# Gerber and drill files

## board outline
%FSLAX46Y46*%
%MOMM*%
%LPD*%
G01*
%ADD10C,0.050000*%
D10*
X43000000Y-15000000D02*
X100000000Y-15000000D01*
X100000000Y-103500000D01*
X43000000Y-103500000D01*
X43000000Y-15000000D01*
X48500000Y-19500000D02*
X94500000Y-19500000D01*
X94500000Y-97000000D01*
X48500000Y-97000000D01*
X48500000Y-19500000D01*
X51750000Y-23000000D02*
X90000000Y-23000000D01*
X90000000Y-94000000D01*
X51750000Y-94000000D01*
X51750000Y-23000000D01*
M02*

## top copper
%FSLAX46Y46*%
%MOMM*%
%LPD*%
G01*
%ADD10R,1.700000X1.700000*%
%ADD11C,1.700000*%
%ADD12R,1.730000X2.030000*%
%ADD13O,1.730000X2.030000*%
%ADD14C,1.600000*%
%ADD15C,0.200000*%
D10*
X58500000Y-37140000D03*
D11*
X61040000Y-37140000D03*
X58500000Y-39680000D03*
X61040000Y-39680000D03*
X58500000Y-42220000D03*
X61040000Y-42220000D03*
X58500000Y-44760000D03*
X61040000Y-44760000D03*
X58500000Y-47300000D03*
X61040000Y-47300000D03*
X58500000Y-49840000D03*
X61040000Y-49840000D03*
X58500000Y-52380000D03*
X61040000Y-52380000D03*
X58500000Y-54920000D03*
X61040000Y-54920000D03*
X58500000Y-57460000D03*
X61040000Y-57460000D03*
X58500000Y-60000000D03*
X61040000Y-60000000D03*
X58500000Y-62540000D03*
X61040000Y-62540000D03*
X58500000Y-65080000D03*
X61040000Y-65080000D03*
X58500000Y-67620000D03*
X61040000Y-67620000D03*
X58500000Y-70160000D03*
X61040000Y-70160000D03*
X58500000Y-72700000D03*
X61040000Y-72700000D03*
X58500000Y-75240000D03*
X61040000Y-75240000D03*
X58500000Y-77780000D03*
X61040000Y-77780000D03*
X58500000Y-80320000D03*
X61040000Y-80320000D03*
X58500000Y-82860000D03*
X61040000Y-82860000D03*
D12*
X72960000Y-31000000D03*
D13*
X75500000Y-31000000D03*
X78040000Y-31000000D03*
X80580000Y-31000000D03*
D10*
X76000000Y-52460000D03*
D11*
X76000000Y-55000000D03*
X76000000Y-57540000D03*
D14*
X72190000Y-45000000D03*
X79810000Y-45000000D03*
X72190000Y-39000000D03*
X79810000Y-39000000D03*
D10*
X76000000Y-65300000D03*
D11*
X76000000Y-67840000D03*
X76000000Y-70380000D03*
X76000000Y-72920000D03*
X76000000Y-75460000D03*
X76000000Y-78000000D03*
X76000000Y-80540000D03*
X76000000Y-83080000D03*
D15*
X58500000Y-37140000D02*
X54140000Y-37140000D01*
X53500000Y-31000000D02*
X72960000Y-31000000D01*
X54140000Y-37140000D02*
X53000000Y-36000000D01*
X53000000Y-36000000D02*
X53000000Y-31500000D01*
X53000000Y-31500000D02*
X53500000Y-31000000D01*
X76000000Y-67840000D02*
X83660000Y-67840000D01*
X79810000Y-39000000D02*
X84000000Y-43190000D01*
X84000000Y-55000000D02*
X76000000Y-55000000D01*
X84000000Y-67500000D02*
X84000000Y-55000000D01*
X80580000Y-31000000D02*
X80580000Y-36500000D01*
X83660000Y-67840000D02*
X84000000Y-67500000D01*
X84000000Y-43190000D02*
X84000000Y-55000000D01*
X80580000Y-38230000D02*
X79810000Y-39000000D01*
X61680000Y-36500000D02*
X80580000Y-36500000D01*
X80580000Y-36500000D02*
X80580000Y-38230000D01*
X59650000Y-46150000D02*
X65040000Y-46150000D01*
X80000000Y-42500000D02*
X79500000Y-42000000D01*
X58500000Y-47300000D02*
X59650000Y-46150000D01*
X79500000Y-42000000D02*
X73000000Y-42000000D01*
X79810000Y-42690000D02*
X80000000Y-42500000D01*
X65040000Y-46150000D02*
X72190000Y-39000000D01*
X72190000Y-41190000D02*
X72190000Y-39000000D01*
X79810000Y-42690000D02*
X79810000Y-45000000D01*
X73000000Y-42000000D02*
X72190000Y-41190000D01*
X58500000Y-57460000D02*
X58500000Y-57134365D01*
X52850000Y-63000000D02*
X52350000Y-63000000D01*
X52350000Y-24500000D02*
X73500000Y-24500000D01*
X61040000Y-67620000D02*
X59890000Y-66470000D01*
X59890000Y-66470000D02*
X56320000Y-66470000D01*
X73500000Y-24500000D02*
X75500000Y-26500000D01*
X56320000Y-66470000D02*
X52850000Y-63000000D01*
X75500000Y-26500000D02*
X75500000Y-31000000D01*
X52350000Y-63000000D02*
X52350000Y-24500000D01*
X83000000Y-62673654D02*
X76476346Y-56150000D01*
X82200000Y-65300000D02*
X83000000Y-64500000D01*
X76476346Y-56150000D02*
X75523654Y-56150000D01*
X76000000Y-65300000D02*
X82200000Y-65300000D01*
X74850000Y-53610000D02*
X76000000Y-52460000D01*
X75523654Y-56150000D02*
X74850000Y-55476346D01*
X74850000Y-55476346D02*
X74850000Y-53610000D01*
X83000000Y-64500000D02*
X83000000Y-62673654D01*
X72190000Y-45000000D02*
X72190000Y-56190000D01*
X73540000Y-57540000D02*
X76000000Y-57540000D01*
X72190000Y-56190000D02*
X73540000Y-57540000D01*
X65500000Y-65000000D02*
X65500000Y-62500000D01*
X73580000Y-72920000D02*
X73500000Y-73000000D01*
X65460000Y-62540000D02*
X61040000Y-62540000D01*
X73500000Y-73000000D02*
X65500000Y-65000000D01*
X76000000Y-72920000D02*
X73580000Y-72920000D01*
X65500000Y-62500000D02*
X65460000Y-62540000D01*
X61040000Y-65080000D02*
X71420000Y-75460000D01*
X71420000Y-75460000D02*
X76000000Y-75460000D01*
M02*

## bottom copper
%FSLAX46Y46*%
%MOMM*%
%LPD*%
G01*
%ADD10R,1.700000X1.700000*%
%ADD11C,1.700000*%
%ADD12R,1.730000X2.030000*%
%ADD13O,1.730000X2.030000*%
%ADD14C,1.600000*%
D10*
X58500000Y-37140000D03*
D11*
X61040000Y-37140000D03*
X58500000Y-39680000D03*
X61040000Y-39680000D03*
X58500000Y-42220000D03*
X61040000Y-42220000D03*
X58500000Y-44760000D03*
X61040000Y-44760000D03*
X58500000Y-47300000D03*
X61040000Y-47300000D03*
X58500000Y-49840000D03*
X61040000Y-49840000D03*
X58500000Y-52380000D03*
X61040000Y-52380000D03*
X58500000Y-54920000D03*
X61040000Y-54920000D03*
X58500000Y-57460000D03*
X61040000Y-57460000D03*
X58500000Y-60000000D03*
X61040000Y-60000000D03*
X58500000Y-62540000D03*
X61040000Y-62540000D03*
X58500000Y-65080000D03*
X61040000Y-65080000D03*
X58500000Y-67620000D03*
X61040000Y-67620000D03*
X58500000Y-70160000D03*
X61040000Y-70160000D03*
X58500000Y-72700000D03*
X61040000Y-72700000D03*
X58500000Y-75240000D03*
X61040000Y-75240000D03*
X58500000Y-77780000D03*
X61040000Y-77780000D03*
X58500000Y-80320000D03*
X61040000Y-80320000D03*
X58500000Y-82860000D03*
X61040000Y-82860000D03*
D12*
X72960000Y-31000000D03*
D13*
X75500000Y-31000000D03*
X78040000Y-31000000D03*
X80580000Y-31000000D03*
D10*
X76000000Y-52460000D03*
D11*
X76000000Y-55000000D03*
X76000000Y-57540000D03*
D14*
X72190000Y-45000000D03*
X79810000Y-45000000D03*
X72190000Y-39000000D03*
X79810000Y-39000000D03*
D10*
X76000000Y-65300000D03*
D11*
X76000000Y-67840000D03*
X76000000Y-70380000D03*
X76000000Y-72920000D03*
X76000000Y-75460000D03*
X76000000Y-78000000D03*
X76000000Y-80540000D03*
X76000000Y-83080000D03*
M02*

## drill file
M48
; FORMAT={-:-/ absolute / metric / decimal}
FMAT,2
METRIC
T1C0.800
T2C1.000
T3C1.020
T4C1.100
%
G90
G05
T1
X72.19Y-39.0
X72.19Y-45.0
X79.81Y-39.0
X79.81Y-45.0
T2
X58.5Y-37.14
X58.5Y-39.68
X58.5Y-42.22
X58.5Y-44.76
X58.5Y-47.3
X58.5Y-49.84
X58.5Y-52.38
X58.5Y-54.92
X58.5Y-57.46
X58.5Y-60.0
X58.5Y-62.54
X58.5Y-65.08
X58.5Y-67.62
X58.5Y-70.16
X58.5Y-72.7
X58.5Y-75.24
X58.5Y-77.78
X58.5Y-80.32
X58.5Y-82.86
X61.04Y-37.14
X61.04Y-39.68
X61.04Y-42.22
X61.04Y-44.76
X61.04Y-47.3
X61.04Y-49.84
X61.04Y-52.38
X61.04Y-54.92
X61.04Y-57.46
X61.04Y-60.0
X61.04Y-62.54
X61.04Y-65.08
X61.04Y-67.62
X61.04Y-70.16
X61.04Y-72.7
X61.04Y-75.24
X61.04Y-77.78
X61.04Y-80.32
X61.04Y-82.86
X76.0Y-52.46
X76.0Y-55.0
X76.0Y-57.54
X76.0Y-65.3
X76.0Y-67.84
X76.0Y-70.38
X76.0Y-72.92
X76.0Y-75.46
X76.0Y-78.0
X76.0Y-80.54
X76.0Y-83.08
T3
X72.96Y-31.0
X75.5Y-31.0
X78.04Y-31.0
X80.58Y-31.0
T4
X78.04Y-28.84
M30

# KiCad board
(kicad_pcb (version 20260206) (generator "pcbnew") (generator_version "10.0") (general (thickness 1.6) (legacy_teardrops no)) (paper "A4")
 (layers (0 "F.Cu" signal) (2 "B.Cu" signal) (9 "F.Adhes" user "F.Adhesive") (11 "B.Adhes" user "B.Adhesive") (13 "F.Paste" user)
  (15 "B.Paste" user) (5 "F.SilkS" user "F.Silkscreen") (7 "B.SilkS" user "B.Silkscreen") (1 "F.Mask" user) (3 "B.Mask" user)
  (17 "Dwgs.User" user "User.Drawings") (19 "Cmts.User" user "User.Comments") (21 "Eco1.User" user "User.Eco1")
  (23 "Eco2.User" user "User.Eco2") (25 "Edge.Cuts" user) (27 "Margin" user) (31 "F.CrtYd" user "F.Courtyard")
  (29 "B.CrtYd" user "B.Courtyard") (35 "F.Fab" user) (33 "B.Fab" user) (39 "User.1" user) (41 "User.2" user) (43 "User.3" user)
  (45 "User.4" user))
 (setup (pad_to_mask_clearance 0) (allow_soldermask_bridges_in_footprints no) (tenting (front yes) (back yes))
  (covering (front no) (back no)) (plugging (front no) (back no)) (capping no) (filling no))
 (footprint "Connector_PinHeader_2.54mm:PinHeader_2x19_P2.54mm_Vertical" (layer "F.Cu") (at 58.5 37.14)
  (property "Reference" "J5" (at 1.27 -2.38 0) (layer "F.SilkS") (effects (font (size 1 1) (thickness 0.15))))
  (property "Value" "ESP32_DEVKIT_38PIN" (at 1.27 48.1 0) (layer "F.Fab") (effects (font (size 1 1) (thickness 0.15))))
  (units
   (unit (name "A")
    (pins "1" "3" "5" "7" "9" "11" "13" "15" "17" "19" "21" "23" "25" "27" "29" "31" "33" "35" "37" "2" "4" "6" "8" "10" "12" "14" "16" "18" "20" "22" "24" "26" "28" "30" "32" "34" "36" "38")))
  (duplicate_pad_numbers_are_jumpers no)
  (pad "1" thru_hole rect (at 0 0) (size 1.7 1.7) (drill 1) (layers "*.Cu" "*.Mask") (remove_unused_layers no) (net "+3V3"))
  (pad "2" thru_hole circle (at 2.54 0) (size 1.7 1.7) (drill 1) (layers "*.Cu" "*.Mask") (remove_unused_layers no) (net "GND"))
  (pad "3" thru_hole circle (at 0 2.54) (size 1.7 1.7) (drill 1) (layers "*.Cu" "*.Mask") (remove_unused_layers no)
   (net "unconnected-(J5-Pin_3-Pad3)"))
  (pad "4" thru_hole circle (at 2.54 2.54) (size 1.7 1.7) (drill 1) (layers "*.Cu" "*.Mask") (remove_unused_layers no)
   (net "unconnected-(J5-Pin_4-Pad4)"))
  (pad "5" thru_hole circle (at 0 5.08) (size 1.7 1.7) (drill 1) (layers "*.Cu" "*.Mask") (remove_unused_layers no)
   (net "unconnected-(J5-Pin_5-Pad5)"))
  (pad "6" thru_hole circle (at 2.54 5.08) (size 1.7 1.7) (drill 1) (layers "*.Cu" "*.Mask") (remove_unused_layers no)
   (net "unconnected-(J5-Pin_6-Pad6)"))
  (pad "7" thru_hole circle (at 0 7.62) (size 1.7 1.7) (drill 1) (layers "*.Cu" "*.Mask") (remove_unused_layers no)
   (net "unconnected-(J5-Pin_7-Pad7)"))
  (pad "8" thru_hole circle (at 2.54 7.62) (size 1.7 1.7) (drill 1) (layers "*.Cu" "*.Mask") (remove_unused_layers no)
   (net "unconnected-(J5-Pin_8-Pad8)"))
  (pad "9" thru_hole circle (at 0 10.16) (size 1.7 1.7) (drill 1) (layers "*.Cu" "*.Mask") (remove_unused_layers no) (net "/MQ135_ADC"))
  (pad "10" thru_hole circle (at 2.54 10.16) (size 1.7 1.7) (drill 1) (layers "*.Cu" "*.Mask") (remove_unused_layers no)
   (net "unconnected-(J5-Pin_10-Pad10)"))
  (pad "11" thru_hole circle (at 0 12.7) (size 1.7 1.7) (drill 1) (layers "*.Cu" "*.Mask") (remove_unused_layers no)
   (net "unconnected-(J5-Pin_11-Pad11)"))
  (pad "12" thru_hole circle (at 2.54 12.7) (size 1.7 1.7) (drill 1) (layers "*.Cu" "*.Mask") (remove_unused_layers no)
   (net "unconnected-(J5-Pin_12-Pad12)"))
  (pad "13" thru_hole circle (at 0 15.24) (size 1.7 1.7) (drill 1) (layers "*.Cu" "*.Mask") (remove_unused_layers no)
   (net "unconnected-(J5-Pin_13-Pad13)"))
  (pad "14" thru_hole circle (at 2.54 15.24) (size 1.7 1.7) (drill 1) (layers "*.Cu" "*.Mask") (remove_unused_layers no)
   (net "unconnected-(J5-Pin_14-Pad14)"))
  (pad "15" thru_hole circle (at 0 17.78) (size 1.7 1.7) (drill 1) (layers "*.Cu" "*.Mask") (remove_unused_layers no)
   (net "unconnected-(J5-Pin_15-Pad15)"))
  (pad "16" thru_hole circle (at 2.54 17.78) (size 1.7 1.7) (drill 1) (layers "*.Cu" "*.Mask") (remove_unused_layers no)
   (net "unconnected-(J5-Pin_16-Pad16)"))
  (pad "17" thru_hole circle (at 0 20.32) (size 1.7 1.7) (drill 1) (layers "*.Cu" "*.Mask") (remove_unused_layers no)
   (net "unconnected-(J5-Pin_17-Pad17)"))
  (pad "18" thru_hole circle (at 2.54 20.32) (size 1.7 1.7) (drill 1) (layers "*.Cu" "*.Mask") (remove_unused_layers no)
   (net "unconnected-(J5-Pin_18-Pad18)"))
  (pad "19" thru_hole circle (at 0 22.86) (size 1.7 1.7) (drill 1) (layers "*.Cu" "*.Mask") (remove_unused_layers no)
   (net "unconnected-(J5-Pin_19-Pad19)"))
  (pad "20" thru_hole circle (at 2.54 22.86) (size 1.7 1.7) (drill 1) (layers "*.Cu" "*.Mask") (remove_unused_layers no)
   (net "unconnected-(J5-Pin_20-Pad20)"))
  (pad "21" thru_hole circle (at 0 25.4) (size 1.7 1.7) (drill 1) (layers "*.Cu" "*.Mask") (remove_unused_layers no)
   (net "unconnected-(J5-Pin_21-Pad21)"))
  (pad "22" thru_hole circle (at 2.54 25.4) (size 1.7 1.7) (drill 1) (layers "*.Cu" "*.Mask") (remove_unused_layers no)
   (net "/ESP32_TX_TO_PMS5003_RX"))
  (pad "23" thru_hole circle (at 0 27.94) (size 1.7 1.7) (drill 1) (layers "*.Cu" "*.Mask") (remove_unused_layers no)
   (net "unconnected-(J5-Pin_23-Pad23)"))
  (pad "24" thru_hole circle (at 2.54 27.94) (size 1.7 1.7) (drill 1) (layers "*.Cu" "*.Mask") (remove_unused_layers no) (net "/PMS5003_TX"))
  (pad "25" thru_hole circle (at 0 30.48) (size 1.7 1.7) (drill 1) (layers "*.Cu" "*.Mask") (remove_unused_layers no)
   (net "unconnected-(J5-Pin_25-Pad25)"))
  (pad "26" thru_hole circle (at 2.54 30.48) (size 1.7 1.7) (drill 1) (layers "*.Cu" "*.Mask") (remove_unused_layers no) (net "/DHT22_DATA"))
  (pad "27" thru_hole circle (at 0 33.02) (size 1.7 1.7) (drill 1) (layers "*.Cu" "*.Mask") (remove_unused_layers no)
   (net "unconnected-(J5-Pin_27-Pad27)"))
  (pad "28" thru_hole circle (at 2.54 33.02) (size 1.7 1.7) (drill 1) (layers "*.Cu" "*.Mask") (remove_unused_layers no)
   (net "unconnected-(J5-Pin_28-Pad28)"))
  (pad "29" thru_hole circle (at 0 35.56) (size 1.7 1.7) (drill 1) (layers "*.Cu" "*.Mask") (remove_unused_layers no)
   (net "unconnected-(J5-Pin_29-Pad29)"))
  (pad "30" thru_hole circle (at 2.54 35.56) (size 1.7 1.7) (drill 1) (layers "*.Cu" "*.Mask") (remove_unused_layers no)
   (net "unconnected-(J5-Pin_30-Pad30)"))
  (pad "31" thru_hole circle (at 0 38.1) (size 1.7 1.7) (drill 1) (layers "*.Cu" "*.Mask") (remove_unused_layers no)
   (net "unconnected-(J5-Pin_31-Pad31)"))
  (pad "32" thru_hole circle (at 2.54 38.1) (size 1.7 1.7) (drill 1) (layers "*.Cu" "*.Mask") (remove_unused_layers no)
   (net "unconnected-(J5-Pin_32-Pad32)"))
  (pad "33" thru_hole circle (at 0 40.64) (size 1.7 1.7) (drill 1) (layers "*.Cu" "*.Mask") (remove_unused_layers no)
   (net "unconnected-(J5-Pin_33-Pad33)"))
  (pad "34" thru_hole circle (at 2.54 40.64) (size 1.7 1.7) (drill 1) (layers "*.Cu" "*.Mask") (remove_unused_layers no)
   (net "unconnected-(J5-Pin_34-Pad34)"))
  (pad "35" thru_hole circle (at 0 43.18) (size 1.7 1.7) (drill 1) (layers "*.Cu" "*.Mask") (remove_unused_layers no)
   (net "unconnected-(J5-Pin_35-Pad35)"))
  (pad "36" thru_hole circle (at 2.54 43.18) (size 1.7 1.7) (drill 1) (layers "*.Cu" "*.Mask") (remove_unused_layers no)
   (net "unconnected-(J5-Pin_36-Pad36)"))
  (pad "37" thru_hole circle (at 0 45.72) (size 1.7 1.7) (drill 1) (layers "*.Cu" "*.Mask") (remove_unused_layers no)
   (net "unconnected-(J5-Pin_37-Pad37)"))
  (pad "38" thru_hole circle (at 2.54 45.72) (size 1.7 1.7) (drill 1) (layers "*.Cu" "*.Mask") (remove_unused_layers no)
   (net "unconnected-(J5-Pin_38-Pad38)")))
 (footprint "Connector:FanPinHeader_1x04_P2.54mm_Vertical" (layer "F.Cu") (at 72.96 31)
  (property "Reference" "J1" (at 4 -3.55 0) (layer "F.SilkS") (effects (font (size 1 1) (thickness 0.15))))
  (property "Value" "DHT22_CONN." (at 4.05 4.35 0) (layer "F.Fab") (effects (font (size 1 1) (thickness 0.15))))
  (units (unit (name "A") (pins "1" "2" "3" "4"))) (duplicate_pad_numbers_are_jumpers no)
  (pad "" np_thru_hole circle (at 5.08 -2.16 90) (size 1.1 1.1) (drill 1.1) (layers "*.Cu" "*.Mask"))
  (pad "1" thru_hole rect (at 0 0 90) (size 2.03 1.73) (drill 1.02) (layers "*.Cu" "*.Mask") (remove_unused_layers no) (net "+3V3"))
  (pad "2" thru_hole oval (at 2.54 0 90) (size 2.03 1.73) (drill 1.02) (layers "*.Cu" "*.Mask") (remove_unused_layers no)
   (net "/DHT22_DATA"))
  (pad "3" thru_hole oval (at 5.08 0 90) (size 2.03 1.73) (drill 1.02) (layers "*.Cu" "*.Mask") (remove_unused_layers no)
   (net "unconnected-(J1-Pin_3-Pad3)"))
  (pad "4" thru_hole oval (at 7.62 0 90) (size 2.03 1.73) (drill 1.02) (layers "*.Cu" "*.Mask") (remove_unused_layers no) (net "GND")))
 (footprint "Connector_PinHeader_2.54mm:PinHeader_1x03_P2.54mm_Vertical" (layer "F.Cu") (at 76 52.46)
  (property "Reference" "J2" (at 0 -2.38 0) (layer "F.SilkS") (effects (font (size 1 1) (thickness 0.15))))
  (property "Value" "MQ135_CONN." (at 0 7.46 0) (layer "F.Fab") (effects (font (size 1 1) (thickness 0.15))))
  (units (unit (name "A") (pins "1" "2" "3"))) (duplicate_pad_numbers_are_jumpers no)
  (pad "1" thru_hole rect (at 0 0) (size 1.7 1.7) (drill 1) (layers "*.Cu" "*.Mask") (remove_unused_layers no) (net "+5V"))
  (pad "2" thru_hole circle (at 0 2.54) (size 1.7 1.7) (drill 1) (layers "*.Cu" "*.Mask") (remove_unused_layers no) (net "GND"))
  (pad "3" thru_hole circle (at 0 5.08) (size 1.7 1.7) (drill 1) (layers "*.Cu" "*.Mask") (remove_unused_layers no) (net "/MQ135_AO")))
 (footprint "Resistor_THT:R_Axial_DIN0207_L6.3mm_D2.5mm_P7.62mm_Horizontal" (layer "F.Cu") (at 72.19 45)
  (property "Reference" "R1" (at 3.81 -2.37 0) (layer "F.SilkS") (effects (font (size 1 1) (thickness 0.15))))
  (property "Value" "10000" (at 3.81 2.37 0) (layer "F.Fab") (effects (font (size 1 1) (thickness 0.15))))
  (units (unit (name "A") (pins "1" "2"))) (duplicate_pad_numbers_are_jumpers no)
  (pad "1" thru_hole circle (at 0 0) (size 1.6 1.6) (drill 0.8) (layers "*.Cu" "*.Mask") (remove_unused_layers no) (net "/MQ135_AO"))
  (pad "2" thru_hole circle (at 7.62 0) (size 1.6 1.6) (drill 0.8) (layers "*.Cu" "*.Mask") (remove_unused_layers no) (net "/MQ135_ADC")))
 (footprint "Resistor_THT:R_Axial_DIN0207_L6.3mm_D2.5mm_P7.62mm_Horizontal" (layer "F.Cu") (at 72.19 39)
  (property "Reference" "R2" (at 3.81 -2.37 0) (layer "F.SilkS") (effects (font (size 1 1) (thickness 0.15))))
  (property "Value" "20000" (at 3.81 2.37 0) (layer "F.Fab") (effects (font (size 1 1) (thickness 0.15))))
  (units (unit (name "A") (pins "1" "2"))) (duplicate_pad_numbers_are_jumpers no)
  (pad "1" thru_hole circle (at 0 0) (size 1.6 1.6) (drill 0.8) (layers "*.Cu" "*.Mask") (remove_unused_layers no) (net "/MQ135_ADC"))
  (pad "2" thru_hole circle (at 7.62 0) (size 1.6 1.6) (drill 0.8) (layers "*.Cu" "*.Mask") (remove_unused_layers no) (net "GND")))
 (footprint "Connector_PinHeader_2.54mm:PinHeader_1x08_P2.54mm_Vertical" (layer "F.Cu") (at 76 65.3)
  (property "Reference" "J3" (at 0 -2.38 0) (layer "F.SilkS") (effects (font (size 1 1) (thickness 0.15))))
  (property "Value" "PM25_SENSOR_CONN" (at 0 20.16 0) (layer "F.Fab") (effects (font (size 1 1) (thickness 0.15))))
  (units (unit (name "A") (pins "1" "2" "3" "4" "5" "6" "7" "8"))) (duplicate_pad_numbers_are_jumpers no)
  (pad "1" thru_hole rect (at 0 0) (size 1.7 1.7) (drill 1) (layers "*.Cu" "*.Mask") (remove_unused_layers no) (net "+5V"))
  (pad "2" thru_hole circle (at 0 2.54) (size 1.7 1.7) (drill 1) (layers "*.Cu" "*.Mask") (remove_unused_layers no) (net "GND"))
  (pad "3" thru_hole circle (at 0 5.08) (size 1.7 1.7) (drill 1) (layers "*.Cu" "*.Mask") (remove_unused_layers no)
   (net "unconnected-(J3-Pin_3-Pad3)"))
  (pad "4" thru_hole circle (at 0 7.62) (size 1.7 1.7) (drill 1) (layers "*.Cu" "*.Mask") (remove_unused_layers no)
   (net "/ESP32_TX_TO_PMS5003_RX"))
  (pad "5" thru_hole circle (at 0 10.16) (size 1.7 1.7) (drill 1) (layers "*.Cu" "*.Mask") (remove_unused_layers no) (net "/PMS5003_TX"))
  (pad "6" thru_hole circle (at 0 12.7) (size 1.7 1.7) (drill 1) (layers "*.Cu" "*.Mask") (remove_unused_layers no)
   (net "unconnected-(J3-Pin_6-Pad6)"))
  (pad "7" thru_hole circle (at 0 15.24) (size 1.7 1.7) (drill 1) (layers "*.Cu" "*.Mask") (remove_unused_layers no)
   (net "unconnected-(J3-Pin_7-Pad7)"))
  (pad "8" thru_hole circle (at 0 17.78) (size 1.7 1.7) (drill 1) (layers "*.Cu" "*.Mask") (remove_unused_layers no)
   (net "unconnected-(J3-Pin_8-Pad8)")))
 (gr_rect (start 43 15) (end 100 103.5) (stroke (width 0.05) (type default)) (fill no) (layer "Edge.Cuts"))
 (gr_rect (start 48.5 19.5) (end 94.5 97) (stroke (width 0.05) (type default)) (fill no) (layer "Edge.Cuts"))
 (gr_rect (start 51.75 23) (end 90 94) (stroke (width 0.05) (type default)) (fill no) (layer "Edge.Cuts"))
 (segment (start 58.5 37.14) (end 54.14 37.14) (width 0.2) (layer "F.Cu") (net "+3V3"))
 (segment (start 53.5 31) (end 72.96 31) (width 0.2) (layer "F.Cu") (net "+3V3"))
 (segment (start 54.14 37.14) (end 53 36) (width 0.2) (layer "F.Cu") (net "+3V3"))
 (segment (start 53 36) (end 53 31.5) (width 0.2) (layer "F.Cu") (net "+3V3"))
 (segment (start 53 31.5) (end 53.5 31) (width 0.2) (layer "F.Cu") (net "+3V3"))
 (segment (start 76 67.84) (end 83.66 67.84) (width 0.2) (layer "F.Cu") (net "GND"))
 (segment (start 79.81 39) (end 84 43.19) (width 0.2) (layer "F.Cu") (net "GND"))
 (segment (start 84 55) (end 76 55) (width 0.2) (layer "F.Cu") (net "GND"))
 (segment (start 84 67.5) (end 84 55) (width 0.2) (layer "F.Cu") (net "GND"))
 (segment (start 80.58 31) (end 80.58 36.5) (width 0.2) (layer "F.Cu") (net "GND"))
 (segment (start 83.66 67.84) (end 84 67.5) (width 0.2) (layer "F.Cu") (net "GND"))
 (segment (start 84 43.19) (end 84 55) (width 0.2) (layer "F.Cu") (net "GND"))
 (segment (start 80.58 38.23) (end 79.81 39) (width 0.2) (layer "F.Cu") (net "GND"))
 (segment (start 61.68 36.5) (end 80.58 36.5) (width 0.2) (layer "F.Cu") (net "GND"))
 (segment (start 80.58 36.5) (end 80.58 38.23) (width 0.2) (layer "F.Cu") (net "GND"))
 (segment (start 59.65 46.15) (end 65.04 46.15) (width 0.2) (layer "F.Cu") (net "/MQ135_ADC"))
 (segment (start 80 42.5) (end 79.5 42) (width 0.2) (layer "F.Cu") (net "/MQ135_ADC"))
 (segment (start 58.5 47.3) (end 59.65 46.15) (width 0.2) (layer "F.Cu") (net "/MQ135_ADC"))
 (segment (start 79.5 42) (end 73 42) (width 0.2) (layer "F.Cu") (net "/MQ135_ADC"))
 (segment (start 79.81 42.69) (end 80 42.5) (width 0.2) (layer "F.Cu") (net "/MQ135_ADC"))
 (segment (start 65.04 46.15) (end 72.19 39) (width 0.2) (layer "F.Cu") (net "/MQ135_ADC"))
 (segment (start 72.19 41.19) (end 72.19 39) (width 0.2) (layer "F.Cu") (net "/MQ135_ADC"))
 (segment (start 79.81 42.69) (end 79.81 45) (width 0.2) (layer "F.Cu") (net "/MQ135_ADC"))
 (segment (start 73 42) (end 72.19 41.19) (width 0.2) (layer "F.Cu") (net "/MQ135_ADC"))
 (segment (start 58.5 57.46) (end 58.5 57.134365) (width 0.2) (layer "F.Cu") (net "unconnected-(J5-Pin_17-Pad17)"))
 (segment (start 52.85 63) (end 52.35 63) (width 0.2) (layer "F.Cu") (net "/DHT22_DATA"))
 (segment (start 52.35 24.5) (end 73.5 24.5) (width 0.2) (layer "F.Cu") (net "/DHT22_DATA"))
 (segment (start 61.04 67.62) (end 59.89 66.47) (width 0.2) (layer "F.Cu") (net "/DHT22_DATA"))
 (segment (start 59.89 66.47) (end 56.32 66.47) (width 0.2) (layer "F.Cu") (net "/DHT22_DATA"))
 (segment (start 73.5 24.5) (end 75.5 26.5) (width 0.2) (layer "F.Cu") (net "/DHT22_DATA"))
 (segment (start 56.32 66.47) (end 52.85 63) (width 0.2) (layer "F.Cu") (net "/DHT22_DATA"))
 (segment (start 75.5 26.5) (end 75.5 31) (width 0.2) (layer "F.Cu") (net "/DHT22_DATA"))
 (segment (start 52.35 63) (end 52.35 24.5) (width 0.2) (layer "F.Cu") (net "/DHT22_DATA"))
 (segment (start 83 62.673654) (end 76.476346 56.15) (width 0.2) (layer "F.Cu") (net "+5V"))
 (segment (start 82.2 65.3) (end 83 64.5) (width 0.2) (layer "F.Cu") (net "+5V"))
 (segment (start 76.476346 56.15) (end 75.523654 56.15) (width 0.2) (layer "F.Cu") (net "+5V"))
 (segment (start 76 65.3) (end 82.2 65.3) (width 0.2) (layer "F.Cu") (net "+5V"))
 (segment (start 74.85 53.61) (end 76 52.46) (width 0.2) (layer "F.Cu") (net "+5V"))
 (segment (start 75.523654 56.15) (end 74.85 55.476346) (width 0.2) (layer "F.Cu") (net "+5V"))
 (segment (start 74.85 55.476346) (end 74.85 53.61) (width 0.2) (layer "F.Cu") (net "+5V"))
 (segment (start 83 64.5) (end 83 62.673654) (width 0.2) (layer "F.Cu") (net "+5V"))
 (segment (start 72.19 45) (end 72.19 56.19) (width 0.2) (layer "F.Cu") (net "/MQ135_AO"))
 (segment (start 73.54 57.54) (end 76 57.54) (width 0.2) (layer "F.Cu") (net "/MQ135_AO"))
 (segment (start 72.19 56.19) (end 73.54 57.54) (width 0.2) (layer "F.Cu") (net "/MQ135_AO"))
 (segment (start 65.5 65) (end 65.5 62.5) (width 0.2) (layer "F.Cu") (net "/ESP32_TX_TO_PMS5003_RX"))
 (segment (start 73.58 72.92) (end 73.5 73) (width 0.2) (layer "F.Cu") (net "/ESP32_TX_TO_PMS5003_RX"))
 (segment (start 65.46 62.54) (end 61.04 62.54) (width 0.2) (layer "F.Cu") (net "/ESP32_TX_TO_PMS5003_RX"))
 (segment (start 73.5 73) (end 65.5 65) (width 0.2) (layer "F.Cu") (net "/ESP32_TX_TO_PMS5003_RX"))
 (segment (start 76 72.92) (end 73.58 72.92) (width 0.2) (layer "F.Cu") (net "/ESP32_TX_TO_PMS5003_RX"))
 (segment (start 65.5 62.5) (end 65.46 62.54) (width 0.2) (layer "F.Cu") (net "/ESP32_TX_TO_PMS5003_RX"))
 (segment (start 61.04 65.08) (end 71.42 75.46) (width 0.2) (layer "F.Cu") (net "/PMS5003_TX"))
 (segment (start 71.42 75.46) (end 76 75.46) (width 0.2) (layer "F.Cu") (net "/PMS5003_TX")))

